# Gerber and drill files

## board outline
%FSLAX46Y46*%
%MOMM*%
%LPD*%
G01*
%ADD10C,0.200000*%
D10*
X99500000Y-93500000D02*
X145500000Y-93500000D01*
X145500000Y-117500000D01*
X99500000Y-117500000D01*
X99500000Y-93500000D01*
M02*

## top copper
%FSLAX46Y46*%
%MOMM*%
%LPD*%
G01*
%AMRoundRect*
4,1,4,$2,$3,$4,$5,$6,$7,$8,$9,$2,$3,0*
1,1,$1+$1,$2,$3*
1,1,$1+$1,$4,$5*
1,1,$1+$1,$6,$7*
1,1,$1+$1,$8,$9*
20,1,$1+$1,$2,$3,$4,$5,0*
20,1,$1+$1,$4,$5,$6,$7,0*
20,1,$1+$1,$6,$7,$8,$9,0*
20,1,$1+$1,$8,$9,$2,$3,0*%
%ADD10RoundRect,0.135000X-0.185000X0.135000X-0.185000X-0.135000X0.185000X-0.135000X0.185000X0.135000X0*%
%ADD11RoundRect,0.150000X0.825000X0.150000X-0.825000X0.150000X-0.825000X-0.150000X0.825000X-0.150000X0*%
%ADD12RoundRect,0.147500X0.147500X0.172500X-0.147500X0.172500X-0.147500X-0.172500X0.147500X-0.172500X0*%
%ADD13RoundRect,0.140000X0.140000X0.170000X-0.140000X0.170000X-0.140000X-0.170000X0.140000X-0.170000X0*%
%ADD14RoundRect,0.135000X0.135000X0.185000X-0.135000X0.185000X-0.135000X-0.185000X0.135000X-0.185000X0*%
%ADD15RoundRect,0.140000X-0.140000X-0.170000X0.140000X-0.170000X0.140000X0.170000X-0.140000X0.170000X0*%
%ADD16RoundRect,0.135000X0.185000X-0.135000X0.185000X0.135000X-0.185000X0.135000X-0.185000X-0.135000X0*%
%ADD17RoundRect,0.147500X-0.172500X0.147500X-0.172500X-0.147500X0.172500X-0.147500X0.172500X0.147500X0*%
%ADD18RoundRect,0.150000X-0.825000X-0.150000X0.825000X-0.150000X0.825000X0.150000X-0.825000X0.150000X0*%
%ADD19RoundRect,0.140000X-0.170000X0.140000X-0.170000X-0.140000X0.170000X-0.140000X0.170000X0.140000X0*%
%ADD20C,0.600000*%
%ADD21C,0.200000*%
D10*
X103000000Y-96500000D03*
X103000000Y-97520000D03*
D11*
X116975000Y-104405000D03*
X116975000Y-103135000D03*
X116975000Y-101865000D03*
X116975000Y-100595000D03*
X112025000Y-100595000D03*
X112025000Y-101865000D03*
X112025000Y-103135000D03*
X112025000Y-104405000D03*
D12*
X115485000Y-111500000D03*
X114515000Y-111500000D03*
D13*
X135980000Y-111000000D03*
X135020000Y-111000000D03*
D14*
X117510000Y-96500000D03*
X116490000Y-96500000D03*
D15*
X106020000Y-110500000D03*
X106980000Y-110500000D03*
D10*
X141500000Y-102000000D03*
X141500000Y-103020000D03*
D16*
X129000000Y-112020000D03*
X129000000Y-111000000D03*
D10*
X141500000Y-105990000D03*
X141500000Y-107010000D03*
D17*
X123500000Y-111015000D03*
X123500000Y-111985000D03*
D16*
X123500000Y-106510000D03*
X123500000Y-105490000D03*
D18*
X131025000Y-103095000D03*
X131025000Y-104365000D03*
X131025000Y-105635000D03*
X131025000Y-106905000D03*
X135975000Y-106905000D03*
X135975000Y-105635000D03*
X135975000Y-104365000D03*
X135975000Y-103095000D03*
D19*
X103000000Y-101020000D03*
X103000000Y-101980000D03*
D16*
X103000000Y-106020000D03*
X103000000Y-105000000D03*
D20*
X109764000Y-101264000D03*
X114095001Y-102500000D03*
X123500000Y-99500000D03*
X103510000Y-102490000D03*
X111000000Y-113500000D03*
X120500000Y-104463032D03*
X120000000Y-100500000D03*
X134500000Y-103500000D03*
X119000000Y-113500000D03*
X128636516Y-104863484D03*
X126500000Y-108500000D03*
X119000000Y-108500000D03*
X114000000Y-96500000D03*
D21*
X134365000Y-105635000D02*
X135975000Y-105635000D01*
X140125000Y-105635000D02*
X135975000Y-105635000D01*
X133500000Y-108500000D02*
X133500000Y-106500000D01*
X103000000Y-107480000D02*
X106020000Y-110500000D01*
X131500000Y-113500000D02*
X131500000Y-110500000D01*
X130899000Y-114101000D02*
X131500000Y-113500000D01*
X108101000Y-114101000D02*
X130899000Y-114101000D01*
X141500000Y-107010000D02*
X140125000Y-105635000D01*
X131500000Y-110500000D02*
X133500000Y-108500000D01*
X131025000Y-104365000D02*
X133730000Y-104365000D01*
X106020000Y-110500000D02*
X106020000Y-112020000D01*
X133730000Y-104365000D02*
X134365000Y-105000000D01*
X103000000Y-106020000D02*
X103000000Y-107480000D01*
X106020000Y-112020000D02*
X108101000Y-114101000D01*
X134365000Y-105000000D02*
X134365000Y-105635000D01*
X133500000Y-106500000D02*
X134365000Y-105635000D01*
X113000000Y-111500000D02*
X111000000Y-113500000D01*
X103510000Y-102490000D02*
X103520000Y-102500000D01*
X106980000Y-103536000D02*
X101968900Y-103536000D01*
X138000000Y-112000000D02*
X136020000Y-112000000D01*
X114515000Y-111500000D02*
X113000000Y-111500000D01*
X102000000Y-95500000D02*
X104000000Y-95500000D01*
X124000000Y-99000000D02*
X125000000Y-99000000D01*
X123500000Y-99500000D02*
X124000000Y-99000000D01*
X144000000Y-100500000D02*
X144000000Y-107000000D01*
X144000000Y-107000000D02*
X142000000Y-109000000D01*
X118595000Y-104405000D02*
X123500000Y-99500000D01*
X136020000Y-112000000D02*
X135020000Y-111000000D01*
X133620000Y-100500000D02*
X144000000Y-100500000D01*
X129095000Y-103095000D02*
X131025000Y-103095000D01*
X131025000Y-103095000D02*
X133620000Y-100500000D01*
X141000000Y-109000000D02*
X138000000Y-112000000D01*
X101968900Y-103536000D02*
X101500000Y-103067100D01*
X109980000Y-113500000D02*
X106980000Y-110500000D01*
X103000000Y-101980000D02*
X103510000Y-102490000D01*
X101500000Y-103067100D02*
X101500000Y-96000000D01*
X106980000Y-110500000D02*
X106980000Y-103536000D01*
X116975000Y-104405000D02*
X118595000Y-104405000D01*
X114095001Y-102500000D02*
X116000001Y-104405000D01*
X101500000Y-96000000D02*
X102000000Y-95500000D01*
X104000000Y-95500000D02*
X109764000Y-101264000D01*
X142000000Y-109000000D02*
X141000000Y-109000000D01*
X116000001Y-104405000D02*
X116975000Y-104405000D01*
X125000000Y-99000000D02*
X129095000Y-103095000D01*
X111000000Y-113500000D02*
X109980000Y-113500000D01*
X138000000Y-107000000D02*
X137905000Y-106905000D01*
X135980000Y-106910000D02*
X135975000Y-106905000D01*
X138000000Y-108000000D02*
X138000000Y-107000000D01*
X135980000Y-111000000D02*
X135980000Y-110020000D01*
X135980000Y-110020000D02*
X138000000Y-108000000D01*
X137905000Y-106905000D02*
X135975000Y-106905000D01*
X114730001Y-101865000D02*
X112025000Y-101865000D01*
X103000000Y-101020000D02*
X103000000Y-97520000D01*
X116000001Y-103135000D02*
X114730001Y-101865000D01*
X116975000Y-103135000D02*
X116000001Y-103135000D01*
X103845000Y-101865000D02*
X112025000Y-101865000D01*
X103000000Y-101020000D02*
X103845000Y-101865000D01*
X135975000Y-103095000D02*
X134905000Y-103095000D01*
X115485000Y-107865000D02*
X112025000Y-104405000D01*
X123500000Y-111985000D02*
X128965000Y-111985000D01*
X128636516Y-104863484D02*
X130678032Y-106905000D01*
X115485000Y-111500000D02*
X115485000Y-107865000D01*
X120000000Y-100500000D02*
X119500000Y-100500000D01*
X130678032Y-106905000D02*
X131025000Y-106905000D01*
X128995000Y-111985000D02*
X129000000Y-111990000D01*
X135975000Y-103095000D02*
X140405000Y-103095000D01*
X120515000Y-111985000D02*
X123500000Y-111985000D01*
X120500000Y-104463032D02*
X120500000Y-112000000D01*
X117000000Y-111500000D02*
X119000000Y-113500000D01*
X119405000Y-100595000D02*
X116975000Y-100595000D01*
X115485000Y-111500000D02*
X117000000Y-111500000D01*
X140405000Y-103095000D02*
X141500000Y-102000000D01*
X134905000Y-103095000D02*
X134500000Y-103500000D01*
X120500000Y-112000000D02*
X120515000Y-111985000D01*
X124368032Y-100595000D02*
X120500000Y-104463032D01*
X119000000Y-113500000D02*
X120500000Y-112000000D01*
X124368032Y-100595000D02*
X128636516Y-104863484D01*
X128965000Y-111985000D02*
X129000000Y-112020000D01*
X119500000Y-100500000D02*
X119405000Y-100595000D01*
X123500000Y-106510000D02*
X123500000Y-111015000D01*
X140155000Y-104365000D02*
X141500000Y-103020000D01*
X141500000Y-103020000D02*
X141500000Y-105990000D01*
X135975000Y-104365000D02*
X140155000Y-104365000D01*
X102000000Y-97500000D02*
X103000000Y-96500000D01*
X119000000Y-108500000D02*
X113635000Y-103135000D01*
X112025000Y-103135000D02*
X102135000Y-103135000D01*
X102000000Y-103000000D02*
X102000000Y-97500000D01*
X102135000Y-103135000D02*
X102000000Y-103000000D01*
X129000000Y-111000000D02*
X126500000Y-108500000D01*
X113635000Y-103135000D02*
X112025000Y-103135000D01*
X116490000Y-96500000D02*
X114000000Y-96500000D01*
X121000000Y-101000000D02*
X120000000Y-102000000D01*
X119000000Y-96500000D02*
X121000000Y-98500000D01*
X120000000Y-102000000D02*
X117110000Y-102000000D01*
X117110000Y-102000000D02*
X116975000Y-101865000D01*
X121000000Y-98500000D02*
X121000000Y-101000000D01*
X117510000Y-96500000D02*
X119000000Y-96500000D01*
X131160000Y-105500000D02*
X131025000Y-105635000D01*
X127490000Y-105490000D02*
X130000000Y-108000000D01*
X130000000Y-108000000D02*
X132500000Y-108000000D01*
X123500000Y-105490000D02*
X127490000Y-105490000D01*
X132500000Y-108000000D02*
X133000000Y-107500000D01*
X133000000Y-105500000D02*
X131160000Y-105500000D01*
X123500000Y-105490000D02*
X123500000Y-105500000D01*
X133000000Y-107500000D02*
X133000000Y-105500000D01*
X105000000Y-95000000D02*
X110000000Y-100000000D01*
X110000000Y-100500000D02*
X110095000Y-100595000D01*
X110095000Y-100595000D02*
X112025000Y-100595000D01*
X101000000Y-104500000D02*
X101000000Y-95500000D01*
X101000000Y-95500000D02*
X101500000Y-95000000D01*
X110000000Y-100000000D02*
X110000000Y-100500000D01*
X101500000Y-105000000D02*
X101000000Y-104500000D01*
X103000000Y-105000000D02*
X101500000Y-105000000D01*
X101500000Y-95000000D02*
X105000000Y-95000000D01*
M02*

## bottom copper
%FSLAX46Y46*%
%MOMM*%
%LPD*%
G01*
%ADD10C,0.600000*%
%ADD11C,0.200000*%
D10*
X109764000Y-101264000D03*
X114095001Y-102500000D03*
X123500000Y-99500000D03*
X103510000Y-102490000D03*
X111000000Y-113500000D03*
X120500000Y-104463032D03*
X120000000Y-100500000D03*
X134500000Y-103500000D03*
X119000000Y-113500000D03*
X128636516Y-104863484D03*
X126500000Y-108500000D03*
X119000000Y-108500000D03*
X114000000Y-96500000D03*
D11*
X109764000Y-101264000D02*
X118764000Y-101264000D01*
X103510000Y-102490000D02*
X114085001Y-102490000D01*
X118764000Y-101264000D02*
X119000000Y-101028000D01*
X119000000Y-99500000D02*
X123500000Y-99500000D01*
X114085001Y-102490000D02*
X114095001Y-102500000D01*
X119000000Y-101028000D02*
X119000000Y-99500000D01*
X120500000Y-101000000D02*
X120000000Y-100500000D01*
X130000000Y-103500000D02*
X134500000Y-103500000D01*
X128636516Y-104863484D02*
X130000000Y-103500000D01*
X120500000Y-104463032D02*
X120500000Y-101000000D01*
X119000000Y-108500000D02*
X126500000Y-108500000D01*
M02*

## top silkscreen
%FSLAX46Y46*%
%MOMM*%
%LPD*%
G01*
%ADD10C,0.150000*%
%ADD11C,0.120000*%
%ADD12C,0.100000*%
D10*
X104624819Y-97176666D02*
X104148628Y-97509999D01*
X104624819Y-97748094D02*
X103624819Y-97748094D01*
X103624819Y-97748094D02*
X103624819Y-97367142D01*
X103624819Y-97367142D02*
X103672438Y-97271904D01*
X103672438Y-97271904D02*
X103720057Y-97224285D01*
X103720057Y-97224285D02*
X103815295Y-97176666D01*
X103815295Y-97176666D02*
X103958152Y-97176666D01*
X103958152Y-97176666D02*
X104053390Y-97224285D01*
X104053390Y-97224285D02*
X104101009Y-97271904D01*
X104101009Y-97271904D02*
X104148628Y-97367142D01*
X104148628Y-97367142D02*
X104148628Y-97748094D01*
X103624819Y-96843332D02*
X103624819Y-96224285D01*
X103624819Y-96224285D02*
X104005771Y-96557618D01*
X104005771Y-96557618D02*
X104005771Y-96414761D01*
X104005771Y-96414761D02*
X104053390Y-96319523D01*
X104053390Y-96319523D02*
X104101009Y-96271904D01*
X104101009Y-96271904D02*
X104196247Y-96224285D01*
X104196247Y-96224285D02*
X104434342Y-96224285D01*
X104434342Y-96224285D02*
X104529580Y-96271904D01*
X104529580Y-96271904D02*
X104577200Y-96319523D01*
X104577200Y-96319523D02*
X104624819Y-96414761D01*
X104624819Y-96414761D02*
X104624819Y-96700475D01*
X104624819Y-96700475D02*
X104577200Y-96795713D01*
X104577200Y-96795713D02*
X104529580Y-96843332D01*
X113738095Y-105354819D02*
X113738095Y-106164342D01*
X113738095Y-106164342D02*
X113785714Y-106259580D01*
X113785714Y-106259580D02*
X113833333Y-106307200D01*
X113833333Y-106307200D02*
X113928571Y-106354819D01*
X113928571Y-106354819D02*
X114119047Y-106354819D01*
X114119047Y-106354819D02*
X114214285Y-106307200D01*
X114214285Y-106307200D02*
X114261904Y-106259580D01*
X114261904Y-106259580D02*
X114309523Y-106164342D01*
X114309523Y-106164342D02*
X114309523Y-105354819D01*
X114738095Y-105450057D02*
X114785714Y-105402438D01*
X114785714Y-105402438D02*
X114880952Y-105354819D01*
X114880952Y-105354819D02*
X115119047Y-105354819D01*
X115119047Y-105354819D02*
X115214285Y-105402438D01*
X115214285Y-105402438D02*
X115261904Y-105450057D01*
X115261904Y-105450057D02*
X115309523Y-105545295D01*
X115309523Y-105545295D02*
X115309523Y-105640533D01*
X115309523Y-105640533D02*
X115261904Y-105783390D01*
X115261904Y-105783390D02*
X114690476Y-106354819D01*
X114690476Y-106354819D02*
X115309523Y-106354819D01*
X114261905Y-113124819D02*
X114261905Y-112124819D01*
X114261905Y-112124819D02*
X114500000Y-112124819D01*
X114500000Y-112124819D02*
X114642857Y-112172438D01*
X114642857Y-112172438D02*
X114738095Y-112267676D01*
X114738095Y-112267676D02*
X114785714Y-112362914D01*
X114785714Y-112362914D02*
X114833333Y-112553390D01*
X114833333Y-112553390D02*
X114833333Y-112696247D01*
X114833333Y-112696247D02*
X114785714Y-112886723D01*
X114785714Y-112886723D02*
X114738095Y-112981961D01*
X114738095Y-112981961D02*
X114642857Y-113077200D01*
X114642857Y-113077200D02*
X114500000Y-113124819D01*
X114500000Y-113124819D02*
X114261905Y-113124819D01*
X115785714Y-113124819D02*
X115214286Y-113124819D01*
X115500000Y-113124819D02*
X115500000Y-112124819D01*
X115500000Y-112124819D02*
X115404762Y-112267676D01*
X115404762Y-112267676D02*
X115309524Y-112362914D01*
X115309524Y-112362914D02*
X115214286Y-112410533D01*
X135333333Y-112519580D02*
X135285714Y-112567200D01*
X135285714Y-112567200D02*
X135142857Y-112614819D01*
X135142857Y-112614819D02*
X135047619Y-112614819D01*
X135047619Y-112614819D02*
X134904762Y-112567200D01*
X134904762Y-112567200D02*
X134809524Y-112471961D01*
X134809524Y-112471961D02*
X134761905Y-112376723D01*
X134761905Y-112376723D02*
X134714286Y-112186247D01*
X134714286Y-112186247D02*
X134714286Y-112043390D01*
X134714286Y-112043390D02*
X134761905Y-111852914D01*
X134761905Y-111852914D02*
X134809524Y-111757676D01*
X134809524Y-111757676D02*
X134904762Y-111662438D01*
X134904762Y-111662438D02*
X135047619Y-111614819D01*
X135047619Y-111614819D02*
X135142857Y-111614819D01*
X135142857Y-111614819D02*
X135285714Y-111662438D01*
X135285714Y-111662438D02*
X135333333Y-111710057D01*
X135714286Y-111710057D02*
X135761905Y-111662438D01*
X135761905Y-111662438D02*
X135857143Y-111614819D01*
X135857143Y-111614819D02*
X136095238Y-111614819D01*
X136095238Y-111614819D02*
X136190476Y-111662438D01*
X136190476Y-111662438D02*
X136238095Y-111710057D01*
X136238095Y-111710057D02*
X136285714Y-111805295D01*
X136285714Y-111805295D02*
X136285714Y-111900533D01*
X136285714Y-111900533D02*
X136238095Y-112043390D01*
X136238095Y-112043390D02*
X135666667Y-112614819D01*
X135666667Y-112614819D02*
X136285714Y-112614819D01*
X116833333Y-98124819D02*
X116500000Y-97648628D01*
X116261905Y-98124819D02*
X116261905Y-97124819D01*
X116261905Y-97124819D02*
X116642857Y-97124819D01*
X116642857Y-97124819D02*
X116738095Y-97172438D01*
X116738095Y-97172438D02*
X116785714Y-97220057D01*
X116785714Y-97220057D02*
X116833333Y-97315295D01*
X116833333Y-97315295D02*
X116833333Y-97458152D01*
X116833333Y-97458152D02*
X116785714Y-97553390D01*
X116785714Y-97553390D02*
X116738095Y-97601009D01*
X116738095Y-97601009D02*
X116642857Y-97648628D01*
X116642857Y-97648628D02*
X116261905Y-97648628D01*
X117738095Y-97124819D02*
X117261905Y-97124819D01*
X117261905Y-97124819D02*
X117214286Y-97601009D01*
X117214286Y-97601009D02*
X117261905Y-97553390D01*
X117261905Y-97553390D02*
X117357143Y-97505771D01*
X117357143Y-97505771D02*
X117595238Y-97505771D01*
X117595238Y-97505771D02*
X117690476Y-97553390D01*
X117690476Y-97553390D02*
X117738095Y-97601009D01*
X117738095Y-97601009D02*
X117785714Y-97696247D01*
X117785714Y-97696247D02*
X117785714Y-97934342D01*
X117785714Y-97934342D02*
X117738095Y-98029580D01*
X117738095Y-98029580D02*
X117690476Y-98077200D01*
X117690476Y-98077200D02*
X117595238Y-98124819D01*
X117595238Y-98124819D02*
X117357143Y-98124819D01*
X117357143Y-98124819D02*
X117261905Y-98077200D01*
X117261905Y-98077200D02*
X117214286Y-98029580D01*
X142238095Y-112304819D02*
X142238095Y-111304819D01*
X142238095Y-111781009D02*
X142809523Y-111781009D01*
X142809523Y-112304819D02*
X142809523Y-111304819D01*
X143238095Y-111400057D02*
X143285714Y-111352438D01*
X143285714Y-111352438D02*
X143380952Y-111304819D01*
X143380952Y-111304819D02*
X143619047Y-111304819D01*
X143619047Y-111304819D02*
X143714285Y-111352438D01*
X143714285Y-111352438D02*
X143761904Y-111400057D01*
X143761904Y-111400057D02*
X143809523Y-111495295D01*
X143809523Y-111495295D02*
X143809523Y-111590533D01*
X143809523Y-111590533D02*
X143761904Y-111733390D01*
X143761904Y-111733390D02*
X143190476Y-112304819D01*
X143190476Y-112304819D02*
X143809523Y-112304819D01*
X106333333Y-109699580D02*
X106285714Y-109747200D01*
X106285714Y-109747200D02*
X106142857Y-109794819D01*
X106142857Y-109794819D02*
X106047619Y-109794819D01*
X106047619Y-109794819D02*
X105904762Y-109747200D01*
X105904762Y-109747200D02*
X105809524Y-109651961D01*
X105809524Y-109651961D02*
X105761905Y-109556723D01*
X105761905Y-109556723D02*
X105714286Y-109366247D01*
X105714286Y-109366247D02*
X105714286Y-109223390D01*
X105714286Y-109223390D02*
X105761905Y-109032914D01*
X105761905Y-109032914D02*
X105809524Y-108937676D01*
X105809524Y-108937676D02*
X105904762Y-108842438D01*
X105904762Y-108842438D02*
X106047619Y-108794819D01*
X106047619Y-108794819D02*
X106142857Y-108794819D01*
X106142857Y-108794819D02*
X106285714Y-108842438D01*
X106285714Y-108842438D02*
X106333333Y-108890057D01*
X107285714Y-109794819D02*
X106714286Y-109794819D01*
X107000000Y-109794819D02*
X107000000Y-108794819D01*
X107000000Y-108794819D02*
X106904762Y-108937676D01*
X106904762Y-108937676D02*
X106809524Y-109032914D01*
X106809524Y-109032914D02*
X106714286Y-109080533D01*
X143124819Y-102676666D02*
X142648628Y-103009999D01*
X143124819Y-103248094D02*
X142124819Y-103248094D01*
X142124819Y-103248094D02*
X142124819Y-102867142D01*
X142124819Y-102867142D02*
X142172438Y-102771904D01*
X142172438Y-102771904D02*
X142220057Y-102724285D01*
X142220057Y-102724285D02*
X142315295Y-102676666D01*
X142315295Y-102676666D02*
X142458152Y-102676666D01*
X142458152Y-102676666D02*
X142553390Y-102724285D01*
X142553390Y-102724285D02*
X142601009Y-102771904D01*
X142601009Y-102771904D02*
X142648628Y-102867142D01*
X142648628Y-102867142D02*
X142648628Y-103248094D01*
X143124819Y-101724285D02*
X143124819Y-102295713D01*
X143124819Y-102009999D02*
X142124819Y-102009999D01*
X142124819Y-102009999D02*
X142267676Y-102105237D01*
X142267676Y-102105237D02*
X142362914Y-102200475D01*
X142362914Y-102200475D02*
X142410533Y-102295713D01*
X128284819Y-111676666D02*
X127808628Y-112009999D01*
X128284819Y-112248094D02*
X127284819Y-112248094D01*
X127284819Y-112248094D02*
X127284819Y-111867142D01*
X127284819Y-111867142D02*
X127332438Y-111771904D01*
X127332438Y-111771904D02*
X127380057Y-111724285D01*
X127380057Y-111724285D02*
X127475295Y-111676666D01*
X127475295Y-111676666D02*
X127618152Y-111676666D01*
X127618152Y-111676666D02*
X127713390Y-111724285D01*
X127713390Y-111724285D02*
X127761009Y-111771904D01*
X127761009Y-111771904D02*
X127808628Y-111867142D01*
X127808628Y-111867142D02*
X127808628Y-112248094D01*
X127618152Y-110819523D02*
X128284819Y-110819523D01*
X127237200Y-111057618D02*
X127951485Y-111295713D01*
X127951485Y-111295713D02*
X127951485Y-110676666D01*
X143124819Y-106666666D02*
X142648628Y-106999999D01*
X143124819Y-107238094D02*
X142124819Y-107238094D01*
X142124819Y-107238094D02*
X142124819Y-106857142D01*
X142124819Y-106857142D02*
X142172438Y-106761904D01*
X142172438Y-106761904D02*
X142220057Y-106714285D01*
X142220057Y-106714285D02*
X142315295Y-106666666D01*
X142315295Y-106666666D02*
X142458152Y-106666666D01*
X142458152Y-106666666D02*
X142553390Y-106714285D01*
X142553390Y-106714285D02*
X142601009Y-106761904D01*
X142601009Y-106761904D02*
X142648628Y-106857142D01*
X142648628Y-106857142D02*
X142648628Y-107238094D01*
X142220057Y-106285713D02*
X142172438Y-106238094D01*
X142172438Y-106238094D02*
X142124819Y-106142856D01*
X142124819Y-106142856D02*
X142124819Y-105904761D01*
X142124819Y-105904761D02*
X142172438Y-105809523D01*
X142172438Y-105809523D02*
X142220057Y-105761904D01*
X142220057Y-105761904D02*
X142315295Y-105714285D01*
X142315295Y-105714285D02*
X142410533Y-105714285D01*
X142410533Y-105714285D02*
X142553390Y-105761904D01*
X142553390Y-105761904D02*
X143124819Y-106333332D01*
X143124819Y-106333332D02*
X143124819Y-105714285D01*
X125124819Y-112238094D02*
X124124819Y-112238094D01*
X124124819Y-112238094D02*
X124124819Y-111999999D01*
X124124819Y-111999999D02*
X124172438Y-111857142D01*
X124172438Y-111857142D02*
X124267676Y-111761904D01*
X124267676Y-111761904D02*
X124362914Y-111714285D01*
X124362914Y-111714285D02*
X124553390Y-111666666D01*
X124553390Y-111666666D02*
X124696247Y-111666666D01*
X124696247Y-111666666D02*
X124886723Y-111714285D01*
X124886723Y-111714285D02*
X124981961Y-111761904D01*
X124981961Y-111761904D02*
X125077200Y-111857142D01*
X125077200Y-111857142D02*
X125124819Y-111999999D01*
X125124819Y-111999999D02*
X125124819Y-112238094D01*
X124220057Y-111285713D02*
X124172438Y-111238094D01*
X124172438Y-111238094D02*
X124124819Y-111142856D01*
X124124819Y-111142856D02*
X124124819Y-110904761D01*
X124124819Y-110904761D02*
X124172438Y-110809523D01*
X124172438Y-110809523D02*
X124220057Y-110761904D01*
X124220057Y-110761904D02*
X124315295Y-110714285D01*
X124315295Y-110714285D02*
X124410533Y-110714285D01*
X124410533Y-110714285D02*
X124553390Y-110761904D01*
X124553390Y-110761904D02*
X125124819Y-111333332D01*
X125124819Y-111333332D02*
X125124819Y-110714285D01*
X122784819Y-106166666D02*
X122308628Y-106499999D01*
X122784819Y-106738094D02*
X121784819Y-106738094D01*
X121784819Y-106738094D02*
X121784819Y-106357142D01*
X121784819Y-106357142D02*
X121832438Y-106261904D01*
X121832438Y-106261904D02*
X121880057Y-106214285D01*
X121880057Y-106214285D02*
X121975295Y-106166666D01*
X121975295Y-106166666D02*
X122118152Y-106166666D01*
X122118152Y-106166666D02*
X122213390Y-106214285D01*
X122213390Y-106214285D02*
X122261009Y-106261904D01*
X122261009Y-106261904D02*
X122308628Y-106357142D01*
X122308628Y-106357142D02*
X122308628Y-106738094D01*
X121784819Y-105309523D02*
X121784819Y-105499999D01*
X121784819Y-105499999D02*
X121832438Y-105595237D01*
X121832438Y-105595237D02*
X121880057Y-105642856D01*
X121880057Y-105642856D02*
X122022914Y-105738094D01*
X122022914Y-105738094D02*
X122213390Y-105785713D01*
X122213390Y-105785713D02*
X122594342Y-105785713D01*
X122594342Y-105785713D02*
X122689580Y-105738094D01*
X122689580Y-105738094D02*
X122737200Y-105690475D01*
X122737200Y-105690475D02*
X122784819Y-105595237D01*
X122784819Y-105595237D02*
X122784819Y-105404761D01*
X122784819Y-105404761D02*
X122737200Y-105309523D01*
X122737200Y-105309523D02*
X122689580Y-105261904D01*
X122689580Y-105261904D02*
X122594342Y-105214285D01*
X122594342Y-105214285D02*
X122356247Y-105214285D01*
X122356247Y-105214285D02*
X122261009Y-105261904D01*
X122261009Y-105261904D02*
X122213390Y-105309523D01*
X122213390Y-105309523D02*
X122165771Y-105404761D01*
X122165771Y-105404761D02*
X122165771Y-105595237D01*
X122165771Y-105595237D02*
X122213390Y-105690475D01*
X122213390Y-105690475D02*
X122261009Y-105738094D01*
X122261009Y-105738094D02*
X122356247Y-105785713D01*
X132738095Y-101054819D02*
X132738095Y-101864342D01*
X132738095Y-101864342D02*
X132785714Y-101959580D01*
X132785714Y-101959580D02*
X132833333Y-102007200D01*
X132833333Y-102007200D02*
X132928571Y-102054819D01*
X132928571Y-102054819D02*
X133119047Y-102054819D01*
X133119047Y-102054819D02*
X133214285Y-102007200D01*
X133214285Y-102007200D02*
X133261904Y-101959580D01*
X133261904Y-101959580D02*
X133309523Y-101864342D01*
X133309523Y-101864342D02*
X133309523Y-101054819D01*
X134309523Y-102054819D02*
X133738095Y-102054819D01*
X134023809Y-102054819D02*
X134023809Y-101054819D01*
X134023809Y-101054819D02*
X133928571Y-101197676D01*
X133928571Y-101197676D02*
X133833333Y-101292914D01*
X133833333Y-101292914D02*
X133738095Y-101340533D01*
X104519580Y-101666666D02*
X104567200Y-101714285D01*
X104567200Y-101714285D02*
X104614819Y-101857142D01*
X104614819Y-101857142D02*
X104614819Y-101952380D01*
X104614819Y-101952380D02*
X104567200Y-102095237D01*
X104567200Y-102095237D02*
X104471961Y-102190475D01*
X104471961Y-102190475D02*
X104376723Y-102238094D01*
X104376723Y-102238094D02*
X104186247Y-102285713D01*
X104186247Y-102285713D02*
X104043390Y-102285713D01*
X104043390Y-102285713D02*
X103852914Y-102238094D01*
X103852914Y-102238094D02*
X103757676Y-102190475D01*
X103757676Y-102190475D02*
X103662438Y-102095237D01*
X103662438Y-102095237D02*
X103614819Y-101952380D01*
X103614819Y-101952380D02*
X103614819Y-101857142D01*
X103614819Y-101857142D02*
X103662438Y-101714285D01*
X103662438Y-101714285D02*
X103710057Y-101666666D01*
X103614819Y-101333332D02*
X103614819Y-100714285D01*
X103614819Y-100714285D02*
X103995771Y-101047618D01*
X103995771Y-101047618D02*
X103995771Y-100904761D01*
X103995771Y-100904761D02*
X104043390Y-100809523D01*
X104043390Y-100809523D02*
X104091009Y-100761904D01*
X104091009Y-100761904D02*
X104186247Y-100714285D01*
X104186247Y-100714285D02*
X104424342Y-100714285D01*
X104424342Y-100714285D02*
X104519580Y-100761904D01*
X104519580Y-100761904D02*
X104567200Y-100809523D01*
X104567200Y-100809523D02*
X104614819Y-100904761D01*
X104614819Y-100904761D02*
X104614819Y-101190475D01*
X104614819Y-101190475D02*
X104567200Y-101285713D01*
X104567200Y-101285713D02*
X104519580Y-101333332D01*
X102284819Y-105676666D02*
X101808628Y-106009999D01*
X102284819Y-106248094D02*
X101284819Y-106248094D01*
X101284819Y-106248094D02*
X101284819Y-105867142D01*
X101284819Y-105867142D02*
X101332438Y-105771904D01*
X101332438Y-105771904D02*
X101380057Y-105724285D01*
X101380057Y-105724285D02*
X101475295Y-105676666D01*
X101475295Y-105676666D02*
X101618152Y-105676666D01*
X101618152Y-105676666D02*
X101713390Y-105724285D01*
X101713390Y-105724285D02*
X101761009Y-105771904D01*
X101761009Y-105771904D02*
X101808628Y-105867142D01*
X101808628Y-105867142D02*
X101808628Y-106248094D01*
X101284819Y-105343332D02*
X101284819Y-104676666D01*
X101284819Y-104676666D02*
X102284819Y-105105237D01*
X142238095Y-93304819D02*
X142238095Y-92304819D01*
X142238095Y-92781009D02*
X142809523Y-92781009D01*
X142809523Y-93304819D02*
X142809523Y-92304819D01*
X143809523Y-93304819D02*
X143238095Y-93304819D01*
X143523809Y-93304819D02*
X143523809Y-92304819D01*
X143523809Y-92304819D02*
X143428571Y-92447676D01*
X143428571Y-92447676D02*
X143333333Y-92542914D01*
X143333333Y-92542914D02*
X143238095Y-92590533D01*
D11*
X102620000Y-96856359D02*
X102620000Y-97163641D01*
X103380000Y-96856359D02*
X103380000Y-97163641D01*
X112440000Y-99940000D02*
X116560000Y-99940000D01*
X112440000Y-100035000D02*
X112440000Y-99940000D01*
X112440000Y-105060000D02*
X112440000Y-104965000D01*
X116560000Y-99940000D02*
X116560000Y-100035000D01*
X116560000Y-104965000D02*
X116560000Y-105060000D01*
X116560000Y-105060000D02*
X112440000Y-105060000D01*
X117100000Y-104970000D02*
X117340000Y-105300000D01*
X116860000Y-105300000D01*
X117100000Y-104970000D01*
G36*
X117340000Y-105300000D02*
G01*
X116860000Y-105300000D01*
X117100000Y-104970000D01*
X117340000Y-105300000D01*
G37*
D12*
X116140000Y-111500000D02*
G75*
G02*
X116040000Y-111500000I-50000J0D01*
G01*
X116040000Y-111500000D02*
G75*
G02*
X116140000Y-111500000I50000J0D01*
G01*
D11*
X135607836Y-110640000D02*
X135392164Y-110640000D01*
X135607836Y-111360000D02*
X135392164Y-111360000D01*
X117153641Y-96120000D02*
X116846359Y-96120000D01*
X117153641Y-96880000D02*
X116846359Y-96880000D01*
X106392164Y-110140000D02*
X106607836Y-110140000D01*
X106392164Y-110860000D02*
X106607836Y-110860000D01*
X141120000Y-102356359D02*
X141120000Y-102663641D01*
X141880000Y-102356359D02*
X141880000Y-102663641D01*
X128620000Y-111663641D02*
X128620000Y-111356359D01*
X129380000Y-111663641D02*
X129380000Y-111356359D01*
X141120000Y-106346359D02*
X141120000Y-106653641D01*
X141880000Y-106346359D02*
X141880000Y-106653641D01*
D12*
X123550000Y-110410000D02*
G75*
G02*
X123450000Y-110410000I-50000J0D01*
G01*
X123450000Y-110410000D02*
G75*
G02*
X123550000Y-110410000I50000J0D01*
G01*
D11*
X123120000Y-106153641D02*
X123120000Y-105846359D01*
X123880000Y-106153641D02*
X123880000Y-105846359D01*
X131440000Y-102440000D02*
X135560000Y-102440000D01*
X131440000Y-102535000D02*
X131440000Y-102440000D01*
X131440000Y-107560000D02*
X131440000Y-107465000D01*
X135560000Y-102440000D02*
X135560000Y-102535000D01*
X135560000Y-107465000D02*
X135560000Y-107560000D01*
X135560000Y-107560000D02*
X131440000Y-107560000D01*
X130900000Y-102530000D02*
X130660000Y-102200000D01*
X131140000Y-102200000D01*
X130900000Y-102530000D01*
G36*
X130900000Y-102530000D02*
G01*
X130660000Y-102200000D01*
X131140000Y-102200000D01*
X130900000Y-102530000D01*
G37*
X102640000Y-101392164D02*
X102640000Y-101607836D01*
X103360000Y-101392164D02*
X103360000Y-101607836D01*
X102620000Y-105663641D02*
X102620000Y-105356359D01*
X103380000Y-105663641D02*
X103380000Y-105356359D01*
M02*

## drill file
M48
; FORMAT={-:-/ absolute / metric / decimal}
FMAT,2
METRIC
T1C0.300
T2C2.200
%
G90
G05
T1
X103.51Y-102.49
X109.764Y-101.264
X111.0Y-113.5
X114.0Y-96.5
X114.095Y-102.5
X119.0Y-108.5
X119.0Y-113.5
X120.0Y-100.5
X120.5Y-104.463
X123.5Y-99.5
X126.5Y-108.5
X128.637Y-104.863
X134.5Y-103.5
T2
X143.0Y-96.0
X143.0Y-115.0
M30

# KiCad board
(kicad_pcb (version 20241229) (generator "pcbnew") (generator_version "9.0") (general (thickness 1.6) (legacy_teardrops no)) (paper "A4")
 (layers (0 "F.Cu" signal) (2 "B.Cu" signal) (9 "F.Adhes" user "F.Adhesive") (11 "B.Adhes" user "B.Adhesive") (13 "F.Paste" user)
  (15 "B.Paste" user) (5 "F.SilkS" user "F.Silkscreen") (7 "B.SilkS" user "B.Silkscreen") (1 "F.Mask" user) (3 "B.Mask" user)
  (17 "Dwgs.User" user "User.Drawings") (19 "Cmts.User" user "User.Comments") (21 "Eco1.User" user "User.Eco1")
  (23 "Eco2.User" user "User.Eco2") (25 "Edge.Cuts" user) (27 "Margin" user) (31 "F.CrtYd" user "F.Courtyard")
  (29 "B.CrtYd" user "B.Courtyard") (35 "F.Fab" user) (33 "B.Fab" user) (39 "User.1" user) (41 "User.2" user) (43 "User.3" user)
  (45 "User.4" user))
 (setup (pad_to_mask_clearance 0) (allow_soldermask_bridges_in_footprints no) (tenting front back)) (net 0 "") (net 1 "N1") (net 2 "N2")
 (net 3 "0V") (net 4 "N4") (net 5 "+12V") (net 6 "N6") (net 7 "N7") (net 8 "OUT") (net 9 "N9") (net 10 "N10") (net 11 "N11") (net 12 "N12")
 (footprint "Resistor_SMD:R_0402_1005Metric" (layer "F.Cu") (at 103 97.01 -90)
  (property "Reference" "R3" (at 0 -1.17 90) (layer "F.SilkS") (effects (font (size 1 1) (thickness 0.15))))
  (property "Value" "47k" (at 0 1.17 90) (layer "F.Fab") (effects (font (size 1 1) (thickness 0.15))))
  (fp_line (start -0.153641 0.38) (end 0.153641 0.38) (stroke (width 0.12) (type solid)) (layer "F.SilkS"))
  (fp_line (start -0.153641 -0.38) (end 0.153641 -0.38) (stroke (width 0.12) (type solid)) (layer "F.SilkS"))
  (pad "1" smd roundrect (at -0.51 0 270) (size 0.54 0.64) (layers "F.Cu" "F.Mask" "F.Paste") (roundrect_rratio 0.25) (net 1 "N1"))
  (pad "2" smd roundrect (at 0.51 0 270) (size 0.54 0.64) (layers "F.Cu" "F.Mask" "F.Paste") (roundrect_rratio 0.25) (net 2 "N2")))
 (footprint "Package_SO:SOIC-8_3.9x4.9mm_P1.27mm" (layer "F.Cu") (at 114.5 102.5 180)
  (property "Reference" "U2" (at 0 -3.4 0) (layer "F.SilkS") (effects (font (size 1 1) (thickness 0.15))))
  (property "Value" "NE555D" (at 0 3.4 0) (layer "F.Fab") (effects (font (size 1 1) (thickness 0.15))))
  (fp_line (start 2.06 2.56) (end -2.06 2.56) (stroke (width 0.12) (type solid)) (layer "F.SilkS"))
  (fp_line (start 2.06 2.465) (end 2.06 2.56) (stroke (width 0.12) (type solid)) (layer "F.SilkS"))
  (fp_line (start 2.06 -2.56) (end 2.06 -2.465) (stroke (width 0.12) (type solid)) (layer "F.SilkS"))
  (fp_line (start -2.06 2.56) (end -2.06 2.465) (stroke (width 0.12) (type solid)) (layer "F.SilkS"))
  (fp_line (start -2.06 -2.465) (end -2.06 -2.56) (stroke (width 0.12) (type solid)) (layer "F.SilkS"))
  (fp_line (start -2.06 -2.56) (end 2.06 -2.56) (stroke (width 0.12) (type solid)) (layer "F.SilkS"))
  (fp_poly (pts (xy -2.6 -2.47) (xy -2.84 -2.8) (xy -2.36 -2.8)) (stroke (width 0.12) (type solid)) (fill yes) (layer "F.SilkS"))
  (pad "1" smd roundrect (at -2.475 -1.905 180) (size 1.95 0.6) (layers "F.Cu" "F.Mask" "F.Paste") (roundrect_rratio 0.25) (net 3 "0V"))
  (pad "2" smd roundrect (at -2.475 -0.635 180) (size 1.95 0.6) (layers "F.Cu" "F.Mask" "F.Paste") (roundrect_rratio 0.25) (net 2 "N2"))
  (pad "3" smd roundrect (at -2.475 0.635 180) (size 1.95 0.6) (layers "F.Cu" "F.Mask" "F.Paste") (roundrect_rratio 0.25) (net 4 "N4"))
  (pad "4" smd roundrect (at -2.475 1.905 180) (size 1.95 0.6) (layers "F.Cu" "F.Mask" "F.Paste") (roundrect_rratio 0.25) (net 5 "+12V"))
  (pad "5" smd roundrect (at 2.475 1.905 180) (size 1.95 0.6) (layers "F.Cu" "F.Mask" "F.Paste") (roundrect_rratio 0.25) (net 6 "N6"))
  (pad "6" smd roundrect (at 2.475 0.635 180) (size 1.95 0.6) (layers "F.Cu" "F.Mask" "F.Paste") (roundrect_rratio 0.25) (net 2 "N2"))
  (pad "7" smd roundrect (at 2.475 -0.635 180) (size 1.95 0.6) (layers "F.Cu" "F.Mask" "F.Paste") (roundrect_rratio 0.25) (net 1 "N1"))
  (pad "8" smd roundrect (at 2.475 -1.905 180) (size 1.95 0.6) (layers "F.Cu" "F.Mask" "F.Paste") (roundrect_rratio 0.25) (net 5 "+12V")))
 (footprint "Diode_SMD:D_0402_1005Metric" (layer "F.Cu") (at 115 111.5 180)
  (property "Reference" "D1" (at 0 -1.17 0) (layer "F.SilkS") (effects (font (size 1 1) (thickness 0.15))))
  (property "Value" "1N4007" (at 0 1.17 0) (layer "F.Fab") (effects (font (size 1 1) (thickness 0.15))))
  (fp_circle (center -1.09 0) (end -1.04 0) (stroke (width 0.1) (type solid)) (fill no) (layer "F.SilkS"))
  (pad "1" smd roundrect (at -0.485 0 180) (size 0.59 0.64) (layers "F.Cu" "F.Mask" "F.Paste") (roundrect_rratio 0.25) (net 5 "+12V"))
  (pad "2" smd roundrect (at 0.485 0 180) (size 0.59 0.64) (layers "F.Cu" "F.Mask" "F.Paste") (roundrect_rratio 0.25) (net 3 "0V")))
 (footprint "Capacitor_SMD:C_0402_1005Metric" (layer "F.Cu") (at 135.5 111 180)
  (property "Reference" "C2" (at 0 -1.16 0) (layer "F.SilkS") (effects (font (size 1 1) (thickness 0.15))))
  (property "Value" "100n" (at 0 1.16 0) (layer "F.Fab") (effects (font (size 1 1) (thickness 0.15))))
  (fp_line (start -0.107836 0.36) (end 0.107836 0.36) (stroke (width 0.12) (type solid)) (layer "F.SilkS"))
  (fp_line (start -0.107836 -0.36) (end 0.107836 -0.36) (stroke (width 0.12) (type solid)) (layer "F.SilkS"))
  (pad "1" smd roundrect (at -0.48 0 180) (size 0.56 0.62) (layers "F.Cu" "F.Mask" "F.Paste") (roundrect_rratio 0.25) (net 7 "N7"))
  (pad "2" smd roundrect (at 0.48 0 180) (size 0.56 0.62) (layers "F.Cu" "F.Mask" "F.Paste") (roundrect_rratio 0.25) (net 3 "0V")))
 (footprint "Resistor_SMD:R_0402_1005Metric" (layer "F.Cu") (at 117 96.5 180)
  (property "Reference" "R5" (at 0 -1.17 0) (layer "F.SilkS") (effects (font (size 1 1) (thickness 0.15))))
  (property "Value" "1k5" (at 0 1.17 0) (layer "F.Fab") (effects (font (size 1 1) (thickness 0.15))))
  (fp_line (start -0.153641 0.38) (end 0.153641 0.38) (stroke (width 0.12) (type solid)) (layer "F.SilkS"))
  (fp_line (start -0.153641 -0.38) (end 0.153641 -0.38) (stroke (width 0.12) (type solid)) (layer "F.SilkS"))
  (pad "1" smd roundrect (at -0.51 0 180) (size 0.54 0.64) (layers "F.Cu" "F.Mask" "F.Paste") (roundrect_rratio 0.25) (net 4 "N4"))
  (pad "2" smd roundrect (at 0.51 0 180) (size 0.54 0.64) (layers "F.Cu" "F.Mask" "F.Paste") (roundrect_rratio 0.25) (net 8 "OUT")))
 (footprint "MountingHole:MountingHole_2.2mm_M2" (layer "F.Cu") (at 143 115)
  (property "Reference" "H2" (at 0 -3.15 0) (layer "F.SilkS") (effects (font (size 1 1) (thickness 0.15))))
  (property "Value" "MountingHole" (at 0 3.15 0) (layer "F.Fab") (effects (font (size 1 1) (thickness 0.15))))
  (pad "" np_thru_hole circle (at 0 0) (size 2.2 2.2) (drill 2.2) (layers "*.Cu" "*.Mask")))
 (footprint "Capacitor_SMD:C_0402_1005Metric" (layer "F.Cu") (at 106.5 110.5)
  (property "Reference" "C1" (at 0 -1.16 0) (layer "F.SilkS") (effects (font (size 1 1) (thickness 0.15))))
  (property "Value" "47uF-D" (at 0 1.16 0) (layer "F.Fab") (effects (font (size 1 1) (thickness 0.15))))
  (fp_line (start -0.107836 -0.36) (end 0.107836 -0.36) (stroke (width 0.12) (type solid)) (layer "F.SilkS"))
  (fp_line (start -0.107836 0.36) (end 0.107836 0.36) (stroke (width 0.12) (type solid)) (layer "F.SilkS"))
  (pad "1" smd roundrect (at -0.48 0) (size 0.56 0.62) (layers "F.Cu" "F.Mask" "F.Paste") (roundrect_rratio 0.25) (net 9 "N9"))
  (pad "2" smd roundrect (at 0.48 0) (size 0.56 0.62) (layers "F.Cu" "F.Mask" "F.Paste") (roundrect_rratio 0.25) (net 3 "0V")))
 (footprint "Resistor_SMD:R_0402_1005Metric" (layer "F.Cu") (at 141.5 102.51 -90)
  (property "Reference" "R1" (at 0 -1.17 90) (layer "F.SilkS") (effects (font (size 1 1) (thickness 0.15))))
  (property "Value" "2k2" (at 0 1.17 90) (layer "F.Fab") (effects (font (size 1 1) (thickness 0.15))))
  (fp_line (start -0.153641 0.38) (end 0.153641 0.38) (stroke (width 0.12) (type solid)) (layer "F.SilkS"))
  (fp_line (start -0.153641 -0.38) (end 0.153641 -0.38) (stroke (width 0.12) (type solid)) (layer "F.SilkS"))
  (pad "1" smd roundrect (at -0.51 0 270) (size 0.54 0.64) (layers "F.Cu" "F.Mask" "F.Paste") (roundrect_rratio 0.25) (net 5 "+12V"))
  (pad "2" smd roundrect (at 0.51 0 270) (size 0.54 0.64) (layers "F.Cu" "F.Mask" "F.Paste") (roundrect_rratio 0.25) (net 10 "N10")))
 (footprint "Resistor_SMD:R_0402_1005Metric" (layer "F.Cu") (at 129 111.51 90)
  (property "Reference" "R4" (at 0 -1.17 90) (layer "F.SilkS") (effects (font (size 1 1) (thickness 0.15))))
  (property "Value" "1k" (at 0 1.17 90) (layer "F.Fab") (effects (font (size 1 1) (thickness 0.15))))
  (fp_line (start -0.153641 -0.38) (end 0.153641 -0.38) (stroke (width 0.12) (type solid)) (layer "F.SilkS"))
  (fp_line (start -0.153641 0.38) (end 0.153641 0.38) (stroke (width 0.12) (type solid)) (layer "F.SilkS"))
  (pad "1" smd roundrect (at -0.51 0 90) (size 0.54 0.64) (layers "F.Cu" "F.Mask" "F.Paste") (roundrect_rratio 0.25) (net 5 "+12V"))
  (pad "2" smd roundrect (at 0.51 0 90) (size 0.54 0.64) (layers "F.Cu" "F.Mask" "F.Paste") (roundrect_rratio 0.25) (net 1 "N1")))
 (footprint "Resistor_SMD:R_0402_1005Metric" (layer "F.Cu") (at 141.5 106.5 -90)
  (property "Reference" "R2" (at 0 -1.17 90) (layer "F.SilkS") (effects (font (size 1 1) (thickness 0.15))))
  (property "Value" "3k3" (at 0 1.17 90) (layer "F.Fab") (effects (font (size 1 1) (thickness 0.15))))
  (fp_line (start -0.153641 0.38) (end 0.153641 0.38) (stroke (width 0.12) (type solid)) (layer "F.SilkS"))
  (fp_line (start -0.153641 -0.38) (end 0.153641 -0.38) (stroke (width 0.12) (type solid)) (layer "F.SilkS"))
  (pad "1" smd roundrect (at -0.51 0 270) (size 0.54 0.64) (layers "F.Cu" "F.Mask" "F.Paste") (roundrect_rratio 0.25) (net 10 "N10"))
  (pad "2" smd roundrect (at 0.51 0 270) (size 0.54 0.64) (layers "F.Cu" "F.Mask" "F.Paste") (roundrect_rratio 0.25) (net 9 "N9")))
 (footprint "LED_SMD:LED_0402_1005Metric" (layer "F.Cu") (at 123.5 111.5 -90)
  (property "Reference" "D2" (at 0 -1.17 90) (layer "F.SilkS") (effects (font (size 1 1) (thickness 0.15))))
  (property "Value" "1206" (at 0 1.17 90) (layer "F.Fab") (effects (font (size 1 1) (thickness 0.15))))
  (fp_circle (center -1.09 0) (end -1.04 0) (stroke (width 0.1) (type solid)) (fill no) (layer "F.SilkS"))
  (pad "1" smd roundrect (at -0.485 0 270) (size 0.59 0.64) (layers "F.Cu" "F.Mask" "F.Paste") (roundrect_rratio 0.25) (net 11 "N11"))
  (pad "2" smd roundrect (at 0.485 0 270) (size 0.59 0.64) (layers "F.Cu" "F.Mask" "F.Paste") (roundrect_rratio 0.25) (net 5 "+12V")))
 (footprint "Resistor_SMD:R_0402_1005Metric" (layer "F.Cu") (at 123.5 106 90)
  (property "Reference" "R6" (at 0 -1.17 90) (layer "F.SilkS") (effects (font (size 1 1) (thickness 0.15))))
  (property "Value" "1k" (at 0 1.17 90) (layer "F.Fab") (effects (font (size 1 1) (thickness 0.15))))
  (fp_line (start -0.153641 -0.38) (end 0.153641 -0.38) (stroke (width 0.12) (type solid)) (layer "F.SilkS"))
  (fp_line (start -0.153641 0.38) (end 0.153641 0.38) (stroke (width 0.12) (type solid)) (layer "F.SilkS"))
  (pad "1" smd roundrect (at -0.51 0 90) (size 0.54 0.64) (layers "F.Cu" "F.Mask" "F.Paste") (roundrect_rratio 0.25) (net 11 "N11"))
  (pad "2" smd roundrect (at 0.51 0 90) (size 0.54 0.64) (layers "F.Cu" "F.Mask" "F.Paste") (roundrect_rratio 0.25) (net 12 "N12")))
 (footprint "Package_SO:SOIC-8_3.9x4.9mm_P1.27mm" (layer "F.Cu") (at 133.5 105)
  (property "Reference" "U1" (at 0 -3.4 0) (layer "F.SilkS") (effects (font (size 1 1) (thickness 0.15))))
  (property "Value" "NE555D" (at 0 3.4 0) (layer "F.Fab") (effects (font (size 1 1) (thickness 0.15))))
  (fp_line (start -2.06 -2.56) (end 2.06 -2.56) (stroke (width 0.12) (type solid)) (layer "F.SilkS"))
  (fp_line (start -2.06 -2.465) (end -2.06 -2.56) (stroke (width 0.12) (type solid)) (layer "F.SilkS"))
  (fp_line (start -2.06 2.56) (end -2.06 2.465) (stroke (width 0.12) (type solid)) (layer "F.SilkS"))
  (fp_line (start 2.06 -2.56) (end 2.06 -2.465) (stroke (width 0.12) (type solid)) (layer "F.SilkS"))
  (fp_line (start 2.06 2.465) (end 2.06 2.56) (stroke (width 0.12) (type solid)) (layer "F.SilkS"))
  (fp_line (start 2.06 2.56) (end -2.06 2.56) (stroke (width 0.12) (type solid)) (layer "F.SilkS"))
  (fp_poly (pts (xy -2.6 -2.47) (xy -2.84 -2.8) (xy -2.36 -2.8)) (stroke (width 0.12) (type solid)) (fill yes) (layer "F.SilkS"))
  (pad "1" smd roundrect (at -2.475 -1.905) (size 1.95 0.6) (layers "F.Cu" "F.Mask" "F.Paste") (roundrect_rratio 0.25) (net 3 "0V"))
  (pad "2" smd roundrect (at -2.475 -0.635) (size 1.95 0.6) (layers "F.Cu" "F.Mask" "F.Paste") (roundrect_rratio 0.25) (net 9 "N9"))
  (pad "3" smd roundrect (at -2.475 0.635) (size 1.95 0.6) (layers "F.Cu" "F.Mask" "F.Paste") (roundrect_rratio 0.25) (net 12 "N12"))
  (pad "4" smd roundrect (at -2.475 1.905) (size 1.95 0.6) (layers "F.Cu" "F.Mask" "F.Paste") (roundrect_rratio 0.25) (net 5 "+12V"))
  (pad "5" smd roundrect (at 2.475 1.905) (size 1.95 0.6) (layers "F.Cu" "F.Mask" "F.Paste") (roundrect_rratio 0.25) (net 7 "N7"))
  (pad "6" smd roundrect (at 2.475 0.635) (size 1.95 0.6) (layers "F.Cu" "F.Mask" "F.Paste") (roundrect_rratio 0.25) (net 9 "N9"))
  (pad "7" smd roundrect (at 2.475 -0.635) (size 1.95 0.6) (layers "F.Cu" "F.Mask" "F.Paste") (roundrect_rratio 0.25) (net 10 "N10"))
  (pad "8" smd roundrect (at 2.475 -1.905) (size 1.95 0.6) (layers "F.Cu" "F.Mask" "F.Paste") (roundrect_rratio 0.25) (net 5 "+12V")))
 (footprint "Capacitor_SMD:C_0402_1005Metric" (layer "F.Cu") (at 103 101.5 -90)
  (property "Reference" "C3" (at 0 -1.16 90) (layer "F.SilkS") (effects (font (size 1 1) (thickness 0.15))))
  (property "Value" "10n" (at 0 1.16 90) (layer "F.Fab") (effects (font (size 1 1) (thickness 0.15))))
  (fp_line (start -0.107836 0.36) (end 0.107836 0.36) (stroke (width 0.12) (type solid)) (layer "F.SilkS"))
  (fp_line (start -0.107836 -0.36) (end 0.107836 -0.36) (stroke (width 0.12) (type solid)) (layer "F.SilkS"))
  (pad "1" smd roundrect (at -0.48 0 270) (size 0.56 0.62) (layers "F.Cu" "F.Mask" "F.Paste") (roundrect_rratio 0.25) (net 2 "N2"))
  (pad "2" smd roundrect (at 0.48 0 270) (size 0.56 0.62) (layers "F.Cu" "F.Mask" "F.Paste") (roundrect_rratio 0.25) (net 3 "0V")))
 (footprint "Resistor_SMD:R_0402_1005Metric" (layer "F.Cu") (at 103 105.51 90)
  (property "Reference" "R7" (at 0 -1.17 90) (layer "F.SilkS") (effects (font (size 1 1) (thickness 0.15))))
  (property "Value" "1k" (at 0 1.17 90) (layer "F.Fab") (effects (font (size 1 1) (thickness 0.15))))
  (fp_line (start -0.153641 -0.38) (end 0.153641 -0.38) (stroke (width 0.12) (type solid)) (layer "F.SilkS"))
  (fp_line (start -0.153641 0.38) (end 0.153641 0.38) (stroke (width 0.12) (type solid)) (layer "F.SilkS"))
  (pad "1" smd roundrect (at -0.51 0 90) (size 0.54 0.64) (layers "F.Cu" "F.Mask" "F.Paste") (roundrect_rratio 0.25) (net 9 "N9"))
  (pad "2" smd roundrect (at 0.51 0 90) (size 0.54 0.64) (layers "F.Cu" "F.Mask" "F.Paste") (roundrect_rratio 0.25) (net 6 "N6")))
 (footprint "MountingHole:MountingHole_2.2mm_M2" (layer "F.Cu") (at 143 96)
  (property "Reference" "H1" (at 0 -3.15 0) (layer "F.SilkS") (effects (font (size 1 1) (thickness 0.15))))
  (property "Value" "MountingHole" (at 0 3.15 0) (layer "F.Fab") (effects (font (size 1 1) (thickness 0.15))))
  (pad "" np_thru_hole circle (at 0 0) (size 2.2 2.2) (drill 2.2) (layers "*.Cu" "*.Mask")))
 (gr_rect (start 99.5 93.5) (end 145.5 117.5) (stroke (width 0.2) (type solid)) (fill no) (layer "Edge.Cuts"))
 (segment (start 134.365 105.635) (end 135.975 105.635) (width 0.2) (layer "F.Cu") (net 9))
 (segment (start 140.125 105.635) (end 135.975 105.635) (width 0.2) (layer "F.Cu") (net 9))
 (segment (start 133.5 108.5) (end 133.5 106.5) (width 0.2) (layer "F.Cu") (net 9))
 (segment (start 103 107.48) (end 106.02 110.5) (width 0.2) (layer "F.Cu") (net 9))
 (segment (start 131.5 113.5) (end 131.5 110.5) (width 0.2) (layer "F.Cu") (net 9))
 (segment (start 130.899 114.101) (end 131.5 113.5) (width 0.2) (layer "F.Cu") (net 9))
 (segment (start 108.101 114.101) (end 130.899 114.101) (width 0.2) (layer "F.Cu") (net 9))
 (segment (start 141.5 107.01) (end 140.125 105.635) (width 0.2) (layer "F.Cu") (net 9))
 (segment (start 131.5 110.5) (end 133.5 108.5) (width 0.2) (layer "F.Cu") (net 9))
 (segment (start 131.025 104.365) (end 133.73 104.365) (width 0.2) (layer "F.Cu") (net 9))
 (segment (start 106.02 110.5) (end 106.02 112.02) (width 0.2) (layer "F.Cu") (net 9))
 (segment (start 133.73 104.365) (end 134.365 105) (width 0.2) (layer "F.Cu") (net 9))
 (segment (start 103 106.02) (end 103 107.48) (width 0.2) (layer "F.Cu") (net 9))
 (segment (start 106.02 112.02) (end 108.101 114.101) (width 0.2) (layer "F.Cu") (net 9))
 (segment (start 134.365 105) (end 134.365 105.635) (width 0.2) (layer "F.Cu") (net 9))
 (segment (start 133.5 106.5) (end 134.365 105.635) (width 0.2) (layer "F.Cu") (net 9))
 (segment (start 113 111.5) (end 111 113.5) (width 0.2) (layer "F.Cu") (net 3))
 (segment (start 103.51 102.49) (end 103.52 102.5) (width 0.2) (layer "F.Cu") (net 3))
 (segment (start 106.98 103.536) (end 101.9689 103.536) (width 0.2) (layer "F.Cu") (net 3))
 (segment (start 138 112) (end 136.02 112) (width 0.2) (layer "F.Cu") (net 3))
 (segment (start 114.515 111.5) (end 113 111.5) (width 0.2) (layer "F.Cu") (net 3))
 (segment (start 102 95.5) (end 104 95.5) (width 0.2) (layer "F.Cu") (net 3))
 (segment (start 124 99) (end 125 99) (width 0.2) (layer "F.Cu") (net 3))
 (segment (start 123.5 99.5) (end 124 99) (width 0.2) (layer "F.Cu") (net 3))
 (segment (start 144 100.5) (end 144 107) (width 0.2) (layer "F.Cu") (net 3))
 (segment (start 144 107) (end 142 109) (width 0.2) (layer "F.Cu") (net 3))
 (segment (start 118.595 104.405) (end 123.5 99.5) (width 0.2) (layer "F.Cu") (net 3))
 (segment (start 136.02 112) (end 135.02 111) (width 0.2) (layer "F.Cu") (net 3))
 (segment (start 133.62 100.5) (end 144 100.5) (width 0.2) (layer "F.Cu") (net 3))
 (segment (start 129.095 103.095) (end 131.025 103.095) (width 0.2) (layer "F.Cu") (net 3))
 (segment (start 131.025 103.095) (end 133.62 100.5) (width 0.2) (layer "F.Cu") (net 3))
 (segment (start 141 109) (end 138 112) (width 0.2) (layer "F.Cu") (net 3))
 (segment (start 101.9689 103.536) (end 101.5 103.0671) (width 0.2) (layer "F.Cu") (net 3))
 (segment (start 109.98 113.5) (end 106.98 110.5) (width 0.2) (layer "F.Cu") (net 3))
 (segment (start 103 101.98) (end 103.51 102.49) (width 0.2) (layer "F.Cu") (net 3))
 (segment (start 101.5 103.0671) (end 101.5 96) (width 0.2) (layer "F.Cu") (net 3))
 (segment (start 106.98 110.5) (end 106.98 103.536) (width 0.2) (layer "F.Cu") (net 3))
 (segment (start 116.975 104.405) (end 118.595 104.405) (width 0.2) (layer "F.Cu") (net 3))
 (segment (start 114.095001 102.5) (end 116.000001 104.405) (width 0.2) (layer "F.Cu") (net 3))
 (segment (start 101.5 96) (end 102 95.5) (width 0.2) (layer "F.Cu") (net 3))
 (segment (start 104 95.5) (end 109.764 101.264) (width 0.2) (layer "F.Cu") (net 3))
 (segment (start 142 109) (end 141 109) (width 0.2) (layer "F.Cu") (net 3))
 (segment (start 116.000001 104.405) (end 116.975 104.405) (width 0.2) (layer "F.Cu") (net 3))
 (segment (start 125 99) (end 129.095 103.095) (width 0.2) (layer "F.Cu") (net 3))
 (segment (start 111 113.5) (end 109.98 113.5) (width 0.2) (layer "F.Cu") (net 3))
 (via (at 109.764 101.264) (size 0.6) (drill 0.3) (layers "F.Cu" "B.Cu") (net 3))
 (via (at 114.095001 102.5) (size 0.6) (drill 0.3) (layers "F.Cu" "B.Cu") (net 3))
 (via (at 123.5 99.5) (size 0.6) (drill 0.3) (layers "F.Cu" "B.Cu") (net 3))
 (via (at 103.51 102.49) (size 0.6) (drill 0.3) (layers "F.Cu" "B.Cu") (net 3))
 (via (at 111 113.5) (size 0.6) (drill 0.3) (layers "F.Cu" "B.Cu") (free yes) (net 3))
 (segment (start 109.764 101.264) (end 118.764 101.264) (width 0.2) (layer "B.Cu") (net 3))
 (segment (start 103.51 102.49) (end 114.085001 102.49) (width 0.2) (layer "B.Cu") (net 3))
 (segment (start 118.764 101.264) (end 119 101.028) (width 0.2) (layer "B.Cu") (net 3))
 (segment (start 119 99.5) (end 123.5 99.5) (width 0.2) (layer "B.Cu") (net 3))
 (segment (start 114.085001 102.49) (end 114.095001 102.5) (width 0.2) (layer "B.Cu") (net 3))
 (segment (start 119 101.028) (end 119 99.5) (width 0.2) (layer "B.Cu") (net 3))
 (segment (start 138 107) (end 137.905 106.905) (width 0.2) (layer "F.Cu") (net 7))
 (segment (start 135.98 106.91) (end 135.975 106.905) (width 0.2) (layer "F.Cu") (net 7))
 (segment (start 138 108) (end 138 107) (width 0.2) (layer "F.Cu") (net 7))
 (segment (start 135.98 111) (end 135.98 110.02) (width 0.2) (layer "F.Cu") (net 7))
 (segment (start 135.98 110.02) (end 138 108) (width 0.2) (layer "F.Cu") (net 7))
 (segment (start 137.905 106.905) (end 135.975 106.905) (width 0.2) (layer "F.Cu") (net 7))
 (segment (start 114.730001 101.865) (end 112.025 101.865) (width 0.2) (layer "F.Cu") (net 2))
 (segment (start 103 101.02) (end 103 97.52) (width 0.2) (layer "F.Cu") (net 2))
 (segment (start 116.000001 103.135) (end 114.730001 101.865) (width 0.2) (layer "F.Cu") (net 2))
 (segment (start 116.975 103.135) (end 116.000001 103.135) (width 0.2) (layer "F.Cu") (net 2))
 (segment (start 103.845 101.865) (end 112.025 101.865) (width 0.2) (layer "F.Cu") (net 2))
 (segment (start 103 101.02) (end 103.845 101.865) (width 0.2) (layer "F.Cu") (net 2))
 (segment (start 135.975 103.095) (end 134.905 103.095) (width 0.2) (layer "F.Cu") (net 5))
 (segment (start 115.485 107.865) (end 112.025 104.405) (width 0.2) (layer "F.Cu") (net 5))
 (segment (start 123.5 111.985) (end 128.965 111.985) (width 0.2) (layer "F.Cu") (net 5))
 (segment (start 128.636516 104.863484) (end 130.678032 106.905) (width 0.2) (layer "F.Cu") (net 5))
 (segment (start 115.485 111.5) (end 115.485 107.865) (width 0.2) (layer "F.Cu") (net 5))
 (segment (start 120 100.5) (end 119.5 100.5) (width 0.2) (layer "F.Cu") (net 5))
 (segment (start 130.678032 106.905) (end 131.025 106.905) (width 0.2) (layer "F.Cu") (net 5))
 (segment (start 128.995 111.985) (end 129 111.99) (width 0.2) (layer "F.Cu") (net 5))
 (segment (start 135.975 103.095) (end 140.405 103.095) (width 0.2) (layer "F.Cu") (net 5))
 (segment (start 120.515 111.985) (end 123.5 111.985) (width 0.2) (layer "F.Cu") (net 5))
 (segment (start 120.5 104.463032) (end 120.5 112) (width 0.2) (layer "F.Cu") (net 5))
 (segment (start 117 111.5) (end 119 113.5) (width 0.2) (layer "F.Cu") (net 5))
 (segment (start 119.405 100.595) (end 116.975 100.595) (width 0.2) (layer "F.Cu") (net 5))
 (segment (start 115.485 111.5) (end 117 111.5) (width 0.2) (layer "F.Cu") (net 5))
 (segment (start 140.405 103.095) (end 141.5 102) (width 0.2) (layer "F.Cu") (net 5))
 (segment (start 134.905 103.095) (end 134.5 103.5) (width 0.2) (layer "F.Cu") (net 5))
 (segment (start 120.5 112) (end 120.515 111.985) (width 0.2) (layer "F.Cu") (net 5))
 (segment (start 124.368032 100.595) (end 120.5 104.463032) (width 0.2) (layer "F.Cu") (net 5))
 (segment (start 119 113.5) (end 120.5 112) (width 0.2) (layer "F.Cu") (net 5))
 (segment (start 124.368032 100.595) (end 128.636516 104.863484) (width 0.2) (layer "F.Cu") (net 5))
 (segment (start 128.965 111.985) (end 129 112.02) (width 0.2) (layer "F.Cu") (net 5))
 (segment (start 119.5 100.5) (end 119.405 100.595) (width 0.2) (layer "F.Cu") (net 5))
 (via (at 120.5 104.463032) (size 0.6) (drill 0.3) (layers "F.Cu" "B.Cu") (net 5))
 (via (at 120 100.5) (size 0.6) (drill 0.3) (layers "F.Cu" "B.Cu") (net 5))
 (via (at 134.5 103.5) (size 0.6) (drill 0.3) (layers "F.Cu" "B.Cu") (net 5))
 (via (at 119 113.5) (size 0.6) (drill 0.3) (layers "F.Cu" "B.Cu") (free yes) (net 5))
 (via (at 128.636516 104.863484) (size 0.6) (drill 0.3) (layers "F.Cu" "B.Cu") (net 5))
 (segment (start 120.5 101) (end 120 100.5) (width 0.2) (layer "B.Cu") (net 5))
 (segment (start 130 103.5) (end 134.5 103.5) (width 0.2) (layer "B.Cu") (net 5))
 (segment (start 128.636516 104.863484) (end 130 103.5) (width 0.2) (layer "B.Cu") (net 5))
 (segment (start 120.5 104.463032) (end 120.5 101) (width 0.2) (layer "B.Cu") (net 5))
 (segment (start 123.5 106.51) (end 123.5 111.015) (width 0.2) (layer "F.Cu") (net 11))
 (segment (start 140.155 104.365) (end 141.5 103.02) (width 0.2) (layer "F.Cu") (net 10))
 (segment (start 141.5 103.02) (end 141.5 105.99) (width 0.2) (layer "F.Cu") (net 10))
 (segment (start 135.975 104.365) (end 140.155 104.365) (width 0.2) (layer "F.Cu") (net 10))
 (segment (start 102 97.5) (end 103 96.5) (width 0.2) (layer "F.Cu") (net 1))
 (segment (start 119 108.5) (end 113.635 103.135) (width 0.2) (layer "F.Cu") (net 1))
 (segment (start 112.025 103.135) (end 102.135 103.135) (width 0.2) (layer "F.Cu") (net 1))
 (segment (start 102 103) (end 102 97.5) (width 0.2) (layer "F.Cu") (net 1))
 (segment (start 102.135 103.135) (end 102 103) (width 0.2) (layer "F.Cu") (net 1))
 (segment (start 129 111) (end 126.5 108.5) (width 0.2) (layer "F.Cu") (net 1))
 (segment (start 113.635 103.135) (end 112.025 103.135) (width 0.2) (layer "F.Cu") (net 1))
 (via (at 126.5 108.5) (size 0.6) (drill 0.3) (layers "F.Cu" "B.Cu") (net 1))
 (via (at 119 108.5) (size 0.6) (drill 0.3) (layers "F.Cu" "B.Cu") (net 1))
 (segment (start 119 108.5) (end 126.5 108.5) (width 0.2) (layer "B.Cu") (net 1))
 (segment (start 116.49 96.5) (end 114 96.5) (width 0.2) (layer "F.Cu") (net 8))
 (via (at 114 96.5) (size 0.6) (drill 0.3) (layers "F.Cu" "B.Cu") (free yes) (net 8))
 (segment (start 121 101) (end 120 102) (width 0.2) (layer "F.Cu") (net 4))
 (segment (start 119 96.5) (end 121 98.5) (width 0.2) (layer "F.Cu") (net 4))
 (segment (start 120 102) (end 117.11 102) (width 0.2) (layer "F.Cu") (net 4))
 (segment (start 117.11 102) (end 116.975 101.865) (width 0.2) (layer "F.Cu") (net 4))
 (segment (start 121 98.5) (end 121 101) (width 0.2) (layer "F.Cu") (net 4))
 (segment (start 117.51 96.5) (end 119 96.5) (width 0.2) (layer "F.Cu") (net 4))
 (segment (start 131.16 105.5) (end 131.025 105.635) (width 0.2) (layer "F.Cu") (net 12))
 (segment (start 127.49 105.49) (end 130 108) (width 0.2) (layer "F.Cu") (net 12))
 (segment (start 130 108) (end 132.5 108) (width 0.2) (layer "F.Cu") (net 12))
 (segment (start 123.5 105.49) (end 127.49 105.49) (width 0.2) (layer "F.Cu") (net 12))
 (segment (start 132.5 108) (end 133 107.5) (width 0.2) (layer "F.Cu") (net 12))
 (segment (start 133 105.5) (end 131.16 105.5) (width 0.2) (layer "F.Cu") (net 12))
 (segment (start 123.5 105.49) (end 123.5 105.5) (width 0.2) (layer "F.Cu") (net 12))
 (segment (start 133 107.5) (end 133 105.5) (width 0.2) (layer "F.Cu") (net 12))
 (segment (start 105 95) (end 110 100) (width 0.2) (layer "F.Cu") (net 6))
 (segment (start 110 100.5) (end 110.095 100.595) (width 0.2) (layer "F.Cu") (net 6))
 (segment (start 110.095 100.595) (end 112.025 100.595) (width 0.2) (layer "F.Cu") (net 6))
 (segment (start 101 104.5) (end 101 95.5) (width 0.2) (layer "F.Cu") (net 6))
 (segment (start 101 95.5) (end 101.5 95) (width 0.2) (layer "F.Cu") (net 6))
 (segment (start 110 100) (end 110 100.5) (width 0.2) (layer "F.Cu") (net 6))
 (segment (start 101.5 105) (end 101 104.5) (width 0.2) (layer "F.Cu") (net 6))
 (segment (start 103 105) (end 101.5 105) (width 0.2) (layer "F.Cu") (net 6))
 (segment (start 101.5 95) (end 105 95) (width 0.2) (layer "F.Cu") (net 6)))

